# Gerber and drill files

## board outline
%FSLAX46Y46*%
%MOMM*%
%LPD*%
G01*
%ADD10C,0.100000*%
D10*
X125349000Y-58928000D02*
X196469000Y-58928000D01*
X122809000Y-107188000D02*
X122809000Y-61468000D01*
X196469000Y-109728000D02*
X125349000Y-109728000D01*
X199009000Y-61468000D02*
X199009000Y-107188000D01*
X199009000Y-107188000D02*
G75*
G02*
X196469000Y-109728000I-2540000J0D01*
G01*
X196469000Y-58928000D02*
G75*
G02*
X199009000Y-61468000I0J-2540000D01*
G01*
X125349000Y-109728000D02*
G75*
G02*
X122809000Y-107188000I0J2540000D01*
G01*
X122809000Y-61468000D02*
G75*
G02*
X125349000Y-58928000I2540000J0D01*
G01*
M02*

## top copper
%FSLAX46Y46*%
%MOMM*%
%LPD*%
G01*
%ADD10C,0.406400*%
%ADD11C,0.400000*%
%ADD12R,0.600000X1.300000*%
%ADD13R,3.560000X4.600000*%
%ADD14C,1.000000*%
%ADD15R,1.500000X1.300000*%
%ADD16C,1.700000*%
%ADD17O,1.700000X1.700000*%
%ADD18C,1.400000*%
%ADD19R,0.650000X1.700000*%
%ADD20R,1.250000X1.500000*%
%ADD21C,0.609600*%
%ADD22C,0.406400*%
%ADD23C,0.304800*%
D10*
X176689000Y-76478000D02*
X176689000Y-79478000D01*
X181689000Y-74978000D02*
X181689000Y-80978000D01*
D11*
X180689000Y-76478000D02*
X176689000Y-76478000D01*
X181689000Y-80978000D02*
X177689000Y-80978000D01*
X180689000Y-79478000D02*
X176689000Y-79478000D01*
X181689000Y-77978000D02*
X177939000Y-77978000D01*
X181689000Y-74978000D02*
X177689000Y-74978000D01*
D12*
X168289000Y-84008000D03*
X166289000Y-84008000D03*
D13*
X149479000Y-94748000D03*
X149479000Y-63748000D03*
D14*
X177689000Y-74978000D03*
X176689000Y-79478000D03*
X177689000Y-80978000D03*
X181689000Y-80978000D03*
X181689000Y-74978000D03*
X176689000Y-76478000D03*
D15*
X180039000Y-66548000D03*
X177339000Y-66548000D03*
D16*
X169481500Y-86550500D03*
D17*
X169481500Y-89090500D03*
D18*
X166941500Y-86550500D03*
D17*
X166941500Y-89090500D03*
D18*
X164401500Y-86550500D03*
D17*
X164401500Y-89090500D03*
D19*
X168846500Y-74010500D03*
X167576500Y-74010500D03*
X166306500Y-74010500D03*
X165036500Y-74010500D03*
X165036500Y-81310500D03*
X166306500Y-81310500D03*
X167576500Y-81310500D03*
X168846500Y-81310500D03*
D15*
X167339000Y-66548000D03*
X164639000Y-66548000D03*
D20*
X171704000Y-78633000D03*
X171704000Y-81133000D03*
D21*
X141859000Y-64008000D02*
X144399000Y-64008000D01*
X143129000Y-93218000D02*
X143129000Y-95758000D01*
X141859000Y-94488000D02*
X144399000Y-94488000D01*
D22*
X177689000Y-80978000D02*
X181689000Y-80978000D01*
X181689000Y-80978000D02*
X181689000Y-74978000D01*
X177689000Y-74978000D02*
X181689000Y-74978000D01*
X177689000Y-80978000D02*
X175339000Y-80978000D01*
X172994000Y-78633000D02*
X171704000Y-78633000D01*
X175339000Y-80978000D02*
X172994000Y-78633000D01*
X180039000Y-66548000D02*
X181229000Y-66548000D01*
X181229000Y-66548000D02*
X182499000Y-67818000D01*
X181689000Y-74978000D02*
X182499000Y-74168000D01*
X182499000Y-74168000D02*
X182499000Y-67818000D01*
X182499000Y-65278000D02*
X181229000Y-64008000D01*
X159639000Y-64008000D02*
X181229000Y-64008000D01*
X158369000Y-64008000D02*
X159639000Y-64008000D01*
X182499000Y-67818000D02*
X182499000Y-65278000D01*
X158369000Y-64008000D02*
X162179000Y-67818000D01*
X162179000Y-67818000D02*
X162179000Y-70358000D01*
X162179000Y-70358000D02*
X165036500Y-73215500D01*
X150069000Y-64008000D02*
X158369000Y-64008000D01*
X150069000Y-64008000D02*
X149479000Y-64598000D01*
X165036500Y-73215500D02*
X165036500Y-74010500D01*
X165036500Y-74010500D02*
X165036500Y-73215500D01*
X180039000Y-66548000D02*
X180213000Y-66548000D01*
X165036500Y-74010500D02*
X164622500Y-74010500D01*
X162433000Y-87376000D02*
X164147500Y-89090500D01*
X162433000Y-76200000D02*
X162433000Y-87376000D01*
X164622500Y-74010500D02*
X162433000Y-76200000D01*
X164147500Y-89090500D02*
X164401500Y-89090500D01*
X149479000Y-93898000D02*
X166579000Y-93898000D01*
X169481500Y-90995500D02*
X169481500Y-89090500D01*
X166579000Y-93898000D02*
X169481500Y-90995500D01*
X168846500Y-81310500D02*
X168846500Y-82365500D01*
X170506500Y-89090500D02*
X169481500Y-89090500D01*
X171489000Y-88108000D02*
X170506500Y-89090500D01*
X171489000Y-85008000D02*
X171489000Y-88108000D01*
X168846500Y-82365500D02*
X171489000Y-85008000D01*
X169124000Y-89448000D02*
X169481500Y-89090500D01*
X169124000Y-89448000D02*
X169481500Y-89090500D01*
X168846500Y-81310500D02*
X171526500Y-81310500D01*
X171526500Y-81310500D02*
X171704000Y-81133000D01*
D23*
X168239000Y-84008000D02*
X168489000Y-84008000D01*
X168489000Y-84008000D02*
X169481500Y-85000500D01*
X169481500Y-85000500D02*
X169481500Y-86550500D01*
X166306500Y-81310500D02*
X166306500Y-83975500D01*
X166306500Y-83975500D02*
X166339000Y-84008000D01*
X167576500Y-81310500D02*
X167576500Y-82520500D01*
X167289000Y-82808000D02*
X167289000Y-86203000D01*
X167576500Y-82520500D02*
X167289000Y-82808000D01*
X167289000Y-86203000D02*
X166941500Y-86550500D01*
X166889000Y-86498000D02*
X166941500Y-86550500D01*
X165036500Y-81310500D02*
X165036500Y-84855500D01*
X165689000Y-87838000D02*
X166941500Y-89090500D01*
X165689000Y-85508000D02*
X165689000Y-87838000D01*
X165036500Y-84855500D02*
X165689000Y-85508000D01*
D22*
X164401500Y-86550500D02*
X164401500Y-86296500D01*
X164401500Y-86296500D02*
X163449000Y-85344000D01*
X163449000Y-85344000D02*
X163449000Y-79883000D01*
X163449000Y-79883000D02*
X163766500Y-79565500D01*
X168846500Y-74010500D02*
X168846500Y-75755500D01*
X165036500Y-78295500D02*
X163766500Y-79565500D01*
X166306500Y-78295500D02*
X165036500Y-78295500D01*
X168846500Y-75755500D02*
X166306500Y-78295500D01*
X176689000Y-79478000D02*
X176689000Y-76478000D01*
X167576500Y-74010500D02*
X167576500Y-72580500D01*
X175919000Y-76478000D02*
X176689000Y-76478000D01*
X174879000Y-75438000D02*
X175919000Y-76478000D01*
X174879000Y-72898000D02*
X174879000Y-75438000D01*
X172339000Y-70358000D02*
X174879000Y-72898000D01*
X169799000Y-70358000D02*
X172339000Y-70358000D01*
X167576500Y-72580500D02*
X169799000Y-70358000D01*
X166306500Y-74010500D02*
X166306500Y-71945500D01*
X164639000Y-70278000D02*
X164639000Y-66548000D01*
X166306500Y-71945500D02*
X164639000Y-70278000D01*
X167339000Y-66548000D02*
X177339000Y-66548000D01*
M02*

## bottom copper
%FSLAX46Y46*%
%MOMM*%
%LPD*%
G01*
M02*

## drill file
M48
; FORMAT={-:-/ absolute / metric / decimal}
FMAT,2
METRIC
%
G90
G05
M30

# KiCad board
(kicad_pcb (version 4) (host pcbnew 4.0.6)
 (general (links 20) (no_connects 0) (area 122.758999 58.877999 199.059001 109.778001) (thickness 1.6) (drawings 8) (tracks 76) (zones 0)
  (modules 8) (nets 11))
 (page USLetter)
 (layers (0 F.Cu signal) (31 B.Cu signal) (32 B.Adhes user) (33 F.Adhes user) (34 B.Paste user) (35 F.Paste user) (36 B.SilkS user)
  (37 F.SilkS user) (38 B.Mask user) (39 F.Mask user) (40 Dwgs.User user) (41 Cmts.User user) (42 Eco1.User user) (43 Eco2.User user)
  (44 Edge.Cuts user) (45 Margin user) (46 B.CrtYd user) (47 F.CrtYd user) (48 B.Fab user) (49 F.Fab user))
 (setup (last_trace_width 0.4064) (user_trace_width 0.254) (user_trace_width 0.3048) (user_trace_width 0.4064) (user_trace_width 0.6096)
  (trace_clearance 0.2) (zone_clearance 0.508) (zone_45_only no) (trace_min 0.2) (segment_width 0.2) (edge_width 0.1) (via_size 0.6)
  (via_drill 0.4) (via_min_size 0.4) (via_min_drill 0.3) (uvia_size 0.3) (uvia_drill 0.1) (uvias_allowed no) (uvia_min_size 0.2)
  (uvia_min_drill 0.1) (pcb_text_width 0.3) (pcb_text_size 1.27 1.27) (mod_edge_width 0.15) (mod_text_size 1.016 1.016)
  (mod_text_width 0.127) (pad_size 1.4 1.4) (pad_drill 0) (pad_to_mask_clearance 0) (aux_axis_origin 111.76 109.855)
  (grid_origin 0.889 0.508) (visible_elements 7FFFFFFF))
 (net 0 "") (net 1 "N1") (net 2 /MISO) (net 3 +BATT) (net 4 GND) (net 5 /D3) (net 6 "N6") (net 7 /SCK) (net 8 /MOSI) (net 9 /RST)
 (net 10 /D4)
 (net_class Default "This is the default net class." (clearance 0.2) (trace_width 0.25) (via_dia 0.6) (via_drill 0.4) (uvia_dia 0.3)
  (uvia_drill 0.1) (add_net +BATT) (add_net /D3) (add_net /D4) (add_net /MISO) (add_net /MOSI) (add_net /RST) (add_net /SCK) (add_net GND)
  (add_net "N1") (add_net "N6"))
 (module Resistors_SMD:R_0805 (layer F.Cu) (at 167.289 84.008 180)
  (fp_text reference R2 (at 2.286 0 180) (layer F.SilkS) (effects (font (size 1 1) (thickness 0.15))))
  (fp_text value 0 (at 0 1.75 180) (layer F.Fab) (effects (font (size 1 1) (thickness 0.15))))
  (pad 1 smd rect (at -1 0 180) (size 0.6 1.3) (layers F.Cu F.Paste F.Mask) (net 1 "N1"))
  (pad 2 smd rect (at 1 0 180) (size 0.6 1.3) (layers F.Cu F.Paste F.Mask) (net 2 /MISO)))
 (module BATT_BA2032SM (layer F.Cu) (at 149.479 79.248 90)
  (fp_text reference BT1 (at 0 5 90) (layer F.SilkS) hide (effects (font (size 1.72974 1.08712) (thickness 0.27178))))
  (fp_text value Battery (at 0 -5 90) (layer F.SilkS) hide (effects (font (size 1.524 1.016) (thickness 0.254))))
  (pad 1 smd rect (at -15.5 0 90) (size 4.6 3.56) (layers F.Cu F.Paste F.Mask) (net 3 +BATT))
  (pad 2 smd rect (at 15.5 0 90) (size 4.6 3.56) (layers F.Cu F.Paste F.Mask) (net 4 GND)))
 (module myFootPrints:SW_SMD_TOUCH (layer F.Cu) (at 178.689 77.978 270)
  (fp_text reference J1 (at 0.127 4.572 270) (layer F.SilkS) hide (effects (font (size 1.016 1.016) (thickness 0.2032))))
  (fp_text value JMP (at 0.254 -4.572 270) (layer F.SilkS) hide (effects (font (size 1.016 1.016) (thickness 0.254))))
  (fp_line (start -1.5 2) (end 1.5 2) (layer F.Cu) (width 0.4064))
  (fp_line (start -3 -3) (end 3 -3) (layer F.Cu) (width 0.4064))
  (fp_line (start -1.5 -2) (end -1.5 2) (layer F.Cu) (width 0.4)) (fp_line (start 3 -3) (end 3 1) (layer F.Cu) (width 0.4))
  (fp_line (start 1.5 -2) (end 1.5 2) (layer F.Cu) (width 0.4)) (fp_line (start 0 -3) (end 0 0.75) (layer F.Cu) (width 0.4))
  (fp_line (start -3 -3) (end -3 1) (layer F.Cu) (width 0.4))
  (pad 1 smd circle (at -3 1 270) (size 1 1) (layers F.Cu F.Paste F.Mask) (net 4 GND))
  (pad 2 smd circle (at 1.5 2 270) (size 1 1) (layers F.Cu F.Paste F.Mask) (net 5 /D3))
  (pad 1 smd circle (at 3 1 270) (size 1 1) (layers F.Cu F.Paste F.Mask) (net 4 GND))
  (pad 1 smd circle (at 3 -3 270) (size 1 1) (layers F.Cu F.Paste F.Mask) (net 4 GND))
  (pad 1 smd circle (at -3 -3 270) (size 1 1) (layers F.Cu F.Paste F.Mask) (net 4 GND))
  (pad 2 smd circle (at -1.5 2 270) (size 1 1) (layers F.Cu F.Paste F.Mask) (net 5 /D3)))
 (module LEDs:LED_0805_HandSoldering (layer F.Cu) (at 178.689 66.548 180)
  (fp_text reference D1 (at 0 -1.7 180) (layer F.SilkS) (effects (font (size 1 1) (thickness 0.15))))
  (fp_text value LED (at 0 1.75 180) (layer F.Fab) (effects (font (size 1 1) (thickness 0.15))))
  (pad 1 smd rect (at -1.35 0 180) (size 1.5 1.3) (layers F.Cu F.Paste F.Mask) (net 4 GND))
  (pad 2 smd rect (at 1.35 0 180) (size 1.5 1.3) (layers F.Cu F.Paste F.Mask) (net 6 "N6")))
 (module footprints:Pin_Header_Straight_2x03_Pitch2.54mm (layer F.Cu) (at 169.4815 86.5505 270)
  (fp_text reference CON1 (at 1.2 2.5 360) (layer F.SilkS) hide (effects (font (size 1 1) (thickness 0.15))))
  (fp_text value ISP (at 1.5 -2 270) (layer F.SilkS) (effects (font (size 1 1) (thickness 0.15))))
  (pad 1 smd circle (at 0 0 270) (size 1.7 1.7) (layers F.Cu F.Paste F.Mask) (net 1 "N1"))
  (pad 2 smd oval (at 2.54 0 270) (size 1.7 1.7) (layers F.Cu F.Paste F.Mask) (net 3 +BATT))
  (pad 3 smd circle (at 0 2.54 270) (size 1.4 1.4) (layers F.Cu F.Paste F.Mask) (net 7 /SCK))
  (pad 4 smd oval (at 2.54 2.54 270) (size 1.7 1.7) (layers F.Cu F.Paste F.Mask) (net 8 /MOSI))
  (pad 5 smd circle (at 0 5.08 270) (size 1.4 1.4) (layers F.Cu F.Paste F.Mask) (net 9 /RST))
  (pad 6 smd oval (at 2.54 5.08 270) (size 1.7 1.7) (layers F.Cu F.Paste F.Mask) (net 4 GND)))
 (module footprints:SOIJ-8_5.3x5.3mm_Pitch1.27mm (layer F.Cu) (at 166.9415 77.6605 270)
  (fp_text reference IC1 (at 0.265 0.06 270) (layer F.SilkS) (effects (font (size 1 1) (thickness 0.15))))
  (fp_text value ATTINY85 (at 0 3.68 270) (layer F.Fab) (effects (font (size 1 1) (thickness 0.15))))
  (pad 1 smd rect (at -3.65 -1.905 270) (size 1.7 0.65) (layers F.Cu F.Paste F.Mask) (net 9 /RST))
  (pad 2 smd rect (at -3.65 -0.635 270) (size 1.7 0.65) (layers F.Cu F.Paste F.Mask) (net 5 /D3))
  (pad 3 smd rect (at -3.65 0.635 270) (size 1.7 0.65) (layers F.Cu F.Paste F.Mask) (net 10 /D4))
  (pad 4 smd rect (at -3.65 1.905 270) (size 1.7 0.65) (layers F.Cu F.Paste F.Mask) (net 4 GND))
  (pad 5 smd rect (at 3.65 1.905 270) (size 1.7 0.65) (layers F.Cu F.Paste F.Mask) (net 8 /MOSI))
  (pad 6 smd rect (at 3.65 0.635 270) (size 1.7 0.65) (layers F.Cu F.Paste F.Mask) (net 2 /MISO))
  (pad 7 smd rect (at 3.65 -0.635 270) (size 1.7 0.65) (layers F.Cu F.Paste F.Mask) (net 7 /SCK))
  (pad 8 smd rect (at 3.65 -1.905 270) (size 1.7 0.65) (layers F.Cu F.Paste F.Mask) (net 3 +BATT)))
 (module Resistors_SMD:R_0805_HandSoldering (layer F.Cu) (at 165.989 66.548 180)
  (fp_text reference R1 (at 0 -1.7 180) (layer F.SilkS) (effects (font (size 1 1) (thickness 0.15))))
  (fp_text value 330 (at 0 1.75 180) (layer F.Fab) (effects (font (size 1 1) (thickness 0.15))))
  (pad 1 smd rect (at -1.35 0 180) (size 1.5 1.3) (layers F.Cu F.Paste F.Mask) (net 6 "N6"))
  (pad 2 smd rect (at 1.35 0 180) (size 1.5 1.3) (layers F.Cu F.Paste F.Mask) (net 10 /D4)))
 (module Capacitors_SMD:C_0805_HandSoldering (layer F.Cu) (at 171.704 79.883 270)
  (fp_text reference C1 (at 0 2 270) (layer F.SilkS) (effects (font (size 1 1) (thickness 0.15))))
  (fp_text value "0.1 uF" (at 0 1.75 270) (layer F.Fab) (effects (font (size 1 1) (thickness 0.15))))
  (pad 1 smd rect (at -1.25 0 270) (size 1.5 1.25) (layers F.Cu F.Paste F.Mask) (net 4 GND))
  (pad 2 smd rect (at 1.25 0 270) (size 1.5 1.25) (layers F.Cu F.Paste F.Mask) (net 3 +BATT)))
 (gr_line (start 125.349 58.928) (end 196.469 58.928) (angle 90) (layer Edge.Cuts) (width 0.1))
 (gr_line (start 122.809 107.188) (end 122.809 61.468) (angle 90) (layer Edge.Cuts) (width 0.1))
 (gr_line (start 196.469 109.728) (end 125.349 109.728) (angle 90) (layer Edge.Cuts) (width 0.1))
 (gr_line (start 199.009 61.468) (end 199.009 107.188) (angle 90) (layer Edge.Cuts) (width 0.1))
 (gr_arc (start 196.469 107.188) (end 199.009 107.188) (angle 90) (layer Edge.Cuts) (width 0.1))
 (gr_arc (start 196.469 61.468) (end 196.469 58.928) (angle 90) (layer Edge.Cuts) (width 0.1))
 (gr_arc (start 125.349 107.188) (end 125.349 109.728) (angle 90) (layer Edge.Cuts) (width 0.1))
 (gr_arc (start 125.349 61.468) (end 122.809 61.468) (angle 90) (layer Edge.Cuts) (width 0.1))
 (segment (start 141.859 64.008) (end 144.399 64.008) (width 0.6096) (layer F.Cu) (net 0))
 (segment (start 143.129 93.218) (end 143.129 95.758) (width 0.6096) (layer F.Cu) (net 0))
 (segment (start 141.859 94.488) (end 144.399 94.488) (width 0.6096) (layer F.Cu) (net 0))
 (segment (start 177.689 80.978) (end 181.689 80.978) (width 0.4064) (layer F.Cu) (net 4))
 (segment (start 181.689 80.978) (end 181.689 74.978) (width 0.4064) (layer F.Cu) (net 4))
 (segment (start 177.689 74.978) (end 181.689 74.978) (width 0.4064) (layer F.Cu) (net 4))
 (segment (start 177.689 80.978) (end 175.339 80.978) (width 0.4064) (layer F.Cu) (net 4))
 (segment (start 172.994 78.633) (end 171.704 78.633) (width 0.4064) (layer F.Cu) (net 4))
 (segment (start 175.339 80.978) (end 172.994 78.633) (width 0.4064) (layer F.Cu) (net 4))
 (segment (start 180.039 66.548) (end 181.229 66.548) (width 0.4064) (layer F.Cu) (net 4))
 (segment (start 181.229 66.548) (end 182.499 67.818) (width 0.4064) (layer F.Cu) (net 4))
 (segment (start 181.689 74.978) (end 182.499 74.168) (width 0.4064) (layer F.Cu) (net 4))
 (segment (start 182.499 74.168) (end 182.499 67.818) (width 0.4064) (layer F.Cu) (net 4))
 (segment (start 182.499 65.278) (end 181.229 64.008) (width 0.4064) (layer F.Cu) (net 4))
 (segment (start 159.639 64.008) (end 181.229 64.008) (width 0.4064) (layer F.Cu) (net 4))
 (segment (start 158.369 64.008) (end 159.639 64.008) (width 0.4064) (layer F.Cu) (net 4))
 (segment (start 182.499 67.818) (end 182.499 65.278) (width 0.4064) (layer F.Cu) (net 4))
 (segment (start 158.369 64.008) (end 162.179 67.818) (width 0.4064) (layer F.Cu) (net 4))
 (segment (start 162.179 67.818) (end 162.179 70.358) (width 0.4064) (layer F.Cu) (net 4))
 (segment (start 162.179 70.358) (end 165.0365 73.2155) (width 0.4064) (layer F.Cu) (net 4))
 (segment (start 150.069 64.008) (end 158.369 64.008) (width 0.4064) (layer F.Cu) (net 4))
 (segment (start 150.069 64.008) (end 149.479 64.598) (width 0.4064) (layer F.Cu) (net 4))
 (segment (start 165.0365 73.2155) (end 165.0365 74.0105) (width 0.4064) (layer F.Cu) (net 4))
 (segment (start 165.0365 74.0105) (end 165.0365 73.2155) (width 0.4064) (layer F.Cu) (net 4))
 (segment (start 180.039 66.548) (end 180.213 66.548) (width 0.4064) (layer F.Cu) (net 4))
 (segment (start 165.0365 74.0105) (end 164.6225 74.0105) (width 0.4064) (layer F.Cu) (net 4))
 (segment (start 162.433 87.376) (end 164.1475 89.0905) (width 0.4064) (layer F.Cu) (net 4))
 (segment (start 162.433 76.2) (end 162.433 87.376) (width 0.4064) (layer F.Cu) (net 4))
 (segment (start 164.6225 74.0105) (end 162.433 76.2) (width 0.4064) (layer F.Cu) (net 4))
 (segment (start 164.1475 89.0905) (end 164.4015 89.0905) (width 0.4064) (layer F.Cu) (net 4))
 (segment (start 149.479 93.898) (end 166.579 93.898) (width 0.4064) (layer F.Cu) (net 3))
 (segment (start 169.4815 90.9955) (end 169.4815 89.0905) (width 0.4064) (layer F.Cu) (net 3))
 (segment (start 166.579 93.898) (end 169.4815 90.9955) (width 0.4064) (layer F.Cu) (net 3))
 (segment (start 168.8465 81.3105) (end 168.8465 82.3655) (width 0.4064) (layer F.Cu) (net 3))
 (segment (start 170.5065 89.0905) (end 169.4815 89.0905) (width 0.4064) (layer F.Cu) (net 3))
 (segment (start 171.489 88.108) (end 170.5065 89.0905) (width 0.4064) (layer F.Cu) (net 3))
 (segment (start 171.489 85.008) (end 171.489 88.108) (width 0.4064) (layer F.Cu) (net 3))
 (segment (start 168.8465 82.3655) (end 171.489 85.008) (width 0.4064) (layer F.Cu) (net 3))
 (segment (start 169.124 89.448) (end 169.4815 89.0905) (width 0.4064) (layer F.Cu) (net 3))
 (segment (start 169.124 89.448) (end 169.4815 89.0905) (width 0.4064) (layer F.Cu) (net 3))
 (segment (start 168.8465 81.3105) (end 171.5265 81.3105) (width 0.4064) (layer F.Cu) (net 3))
 (segment (start 171.5265 81.3105) (end 171.704 81.133) (width 0.4064) (layer F.Cu) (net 3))
 (segment (start 168.239 84.008) (end 168.489 84.008) (width 0.3048) (layer F.Cu) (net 1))
 (segment (start 168.489 84.008) (end 169.4815 85.0005) (width 0.3048) (layer F.Cu) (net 1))
 (segment (start 169.4815 85.0005) (end 169.4815 86.5505) (width 0.3048) (layer F.Cu) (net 1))
 (segment (start 166.3065 81.3105) (end 166.3065 83.9755) (width 0.3048) (layer F.Cu) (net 2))
 (segment (start 166.3065 83.9755) (end 166.339 84.008) (width 0.3048) (layer F.Cu) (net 2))
 (segment (start 167.5765 81.3105) (end 167.5765 82.5205) (width 0.3048) (layer F.Cu) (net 7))
 (segment (start 167.289 82.808) (end 167.289 86.203) (width 0.3048) (layer F.Cu) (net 7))
 (segment (start 167.5765 82.5205) (end 167.289 82.808) (width 0.3048) (layer F.Cu) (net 7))
 (segment (start 167.289 86.203) (end 166.9415 86.5505) (width 0.3048) (layer F.Cu) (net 7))
 (segment (start 166.889 86.498) (end 166.9415 86.5505) (width 0.3048) (layer F.Cu) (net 7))
 (segment (start 165.0365 81.3105) (end 165.0365 84.8555) (width 0.3048) (layer F.Cu) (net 8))
 (segment (start 165.689 87.838) (end 166.9415 89.0905) (width 0.3048) (layer F.Cu) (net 8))
 (segment (start 165.689 85.508) (end 165.689 87.838) (width 0.3048) (layer F.Cu) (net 8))
 (segment (start 165.0365 84.8555) (end 165.689 85.508) (width 0.3048) (layer F.Cu) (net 8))
 (segment (start 164.4015 86.5505) (end 164.4015 86.2965) (width 0.4064) (layer F.Cu) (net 9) (status C00000))
 (segment (start 164.4015 86.2965) (end 163.449 85.344) (width 0.4064) (layer F.Cu) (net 9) (status 400000))
 (segment (start 163.449 85.344) (end 163.449 79.883) (width 0.4064) (layer F.Cu) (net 9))
 (segment (start 163.449 79.883) (end 163.7665 79.5655) (width 0.4064) (layer F.Cu) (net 9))
 (segment (start 168.8465 74.0105) (end 168.8465 75.7555) (width 0.4064) (layer F.Cu) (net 9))
 (segment (start 165.0365 78.2955) (end 163.7665 79.5655) (width 0.4064) (layer F.Cu) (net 9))
 (segment (start 166.3065 78.2955) (end 165.0365 78.2955) (width 0.4064) (layer F.Cu) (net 9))
 (segment (start 168.8465 75.7555) (end 166.3065 78.2955) (width 0.4064) (layer F.Cu) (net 9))
 (segment (start 176.689 79.478) (end 176.689 76.478) (width 0.4064) (layer F.Cu) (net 5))
 (segment (start 167.5765 74.0105) (end 167.5765 72.5805) (width 0.4064) (layer F.Cu) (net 5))
 (segment (start 175.919 76.478) (end 176.689 76.478) (width 0.4064) (layer F.Cu) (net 5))
 (segment (start 174.879 75.438) (end 175.919 76.478) (width 0.4064) (layer F.Cu) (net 5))
 (segment (start 174.879 72.898) (end 174.879 75.438) (width 0.4064) (layer F.Cu) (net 5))
 (segment (start 172.339 70.358) (end 174.879 72.898) (width 0.4064) (layer F.Cu) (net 5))
 (segment (start 169.799 70.358) (end 172.339 70.358) (width 0.4064) (layer F.Cu) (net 5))
 (segment (start 167.5765 72.5805) (end 169.799 70.358) (width 0.4064) (layer F.Cu) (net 5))
 (segment (start 166.3065 74.0105) (end 166.3065 71.9455) (width 0.4064) (layer F.Cu) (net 10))
 (segment (start 164.639 70.278) (end 164.639 66.548) (width 0.4064) (layer F.Cu) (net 10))
 (segment (start 166.3065 71.9455) (end 164.639 70.278) (width 0.4064) (layer F.Cu) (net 10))
 (segment (start 167.339 66.548) (end 177.339 66.548) (width 0.4064) (layer F.Cu) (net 6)))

